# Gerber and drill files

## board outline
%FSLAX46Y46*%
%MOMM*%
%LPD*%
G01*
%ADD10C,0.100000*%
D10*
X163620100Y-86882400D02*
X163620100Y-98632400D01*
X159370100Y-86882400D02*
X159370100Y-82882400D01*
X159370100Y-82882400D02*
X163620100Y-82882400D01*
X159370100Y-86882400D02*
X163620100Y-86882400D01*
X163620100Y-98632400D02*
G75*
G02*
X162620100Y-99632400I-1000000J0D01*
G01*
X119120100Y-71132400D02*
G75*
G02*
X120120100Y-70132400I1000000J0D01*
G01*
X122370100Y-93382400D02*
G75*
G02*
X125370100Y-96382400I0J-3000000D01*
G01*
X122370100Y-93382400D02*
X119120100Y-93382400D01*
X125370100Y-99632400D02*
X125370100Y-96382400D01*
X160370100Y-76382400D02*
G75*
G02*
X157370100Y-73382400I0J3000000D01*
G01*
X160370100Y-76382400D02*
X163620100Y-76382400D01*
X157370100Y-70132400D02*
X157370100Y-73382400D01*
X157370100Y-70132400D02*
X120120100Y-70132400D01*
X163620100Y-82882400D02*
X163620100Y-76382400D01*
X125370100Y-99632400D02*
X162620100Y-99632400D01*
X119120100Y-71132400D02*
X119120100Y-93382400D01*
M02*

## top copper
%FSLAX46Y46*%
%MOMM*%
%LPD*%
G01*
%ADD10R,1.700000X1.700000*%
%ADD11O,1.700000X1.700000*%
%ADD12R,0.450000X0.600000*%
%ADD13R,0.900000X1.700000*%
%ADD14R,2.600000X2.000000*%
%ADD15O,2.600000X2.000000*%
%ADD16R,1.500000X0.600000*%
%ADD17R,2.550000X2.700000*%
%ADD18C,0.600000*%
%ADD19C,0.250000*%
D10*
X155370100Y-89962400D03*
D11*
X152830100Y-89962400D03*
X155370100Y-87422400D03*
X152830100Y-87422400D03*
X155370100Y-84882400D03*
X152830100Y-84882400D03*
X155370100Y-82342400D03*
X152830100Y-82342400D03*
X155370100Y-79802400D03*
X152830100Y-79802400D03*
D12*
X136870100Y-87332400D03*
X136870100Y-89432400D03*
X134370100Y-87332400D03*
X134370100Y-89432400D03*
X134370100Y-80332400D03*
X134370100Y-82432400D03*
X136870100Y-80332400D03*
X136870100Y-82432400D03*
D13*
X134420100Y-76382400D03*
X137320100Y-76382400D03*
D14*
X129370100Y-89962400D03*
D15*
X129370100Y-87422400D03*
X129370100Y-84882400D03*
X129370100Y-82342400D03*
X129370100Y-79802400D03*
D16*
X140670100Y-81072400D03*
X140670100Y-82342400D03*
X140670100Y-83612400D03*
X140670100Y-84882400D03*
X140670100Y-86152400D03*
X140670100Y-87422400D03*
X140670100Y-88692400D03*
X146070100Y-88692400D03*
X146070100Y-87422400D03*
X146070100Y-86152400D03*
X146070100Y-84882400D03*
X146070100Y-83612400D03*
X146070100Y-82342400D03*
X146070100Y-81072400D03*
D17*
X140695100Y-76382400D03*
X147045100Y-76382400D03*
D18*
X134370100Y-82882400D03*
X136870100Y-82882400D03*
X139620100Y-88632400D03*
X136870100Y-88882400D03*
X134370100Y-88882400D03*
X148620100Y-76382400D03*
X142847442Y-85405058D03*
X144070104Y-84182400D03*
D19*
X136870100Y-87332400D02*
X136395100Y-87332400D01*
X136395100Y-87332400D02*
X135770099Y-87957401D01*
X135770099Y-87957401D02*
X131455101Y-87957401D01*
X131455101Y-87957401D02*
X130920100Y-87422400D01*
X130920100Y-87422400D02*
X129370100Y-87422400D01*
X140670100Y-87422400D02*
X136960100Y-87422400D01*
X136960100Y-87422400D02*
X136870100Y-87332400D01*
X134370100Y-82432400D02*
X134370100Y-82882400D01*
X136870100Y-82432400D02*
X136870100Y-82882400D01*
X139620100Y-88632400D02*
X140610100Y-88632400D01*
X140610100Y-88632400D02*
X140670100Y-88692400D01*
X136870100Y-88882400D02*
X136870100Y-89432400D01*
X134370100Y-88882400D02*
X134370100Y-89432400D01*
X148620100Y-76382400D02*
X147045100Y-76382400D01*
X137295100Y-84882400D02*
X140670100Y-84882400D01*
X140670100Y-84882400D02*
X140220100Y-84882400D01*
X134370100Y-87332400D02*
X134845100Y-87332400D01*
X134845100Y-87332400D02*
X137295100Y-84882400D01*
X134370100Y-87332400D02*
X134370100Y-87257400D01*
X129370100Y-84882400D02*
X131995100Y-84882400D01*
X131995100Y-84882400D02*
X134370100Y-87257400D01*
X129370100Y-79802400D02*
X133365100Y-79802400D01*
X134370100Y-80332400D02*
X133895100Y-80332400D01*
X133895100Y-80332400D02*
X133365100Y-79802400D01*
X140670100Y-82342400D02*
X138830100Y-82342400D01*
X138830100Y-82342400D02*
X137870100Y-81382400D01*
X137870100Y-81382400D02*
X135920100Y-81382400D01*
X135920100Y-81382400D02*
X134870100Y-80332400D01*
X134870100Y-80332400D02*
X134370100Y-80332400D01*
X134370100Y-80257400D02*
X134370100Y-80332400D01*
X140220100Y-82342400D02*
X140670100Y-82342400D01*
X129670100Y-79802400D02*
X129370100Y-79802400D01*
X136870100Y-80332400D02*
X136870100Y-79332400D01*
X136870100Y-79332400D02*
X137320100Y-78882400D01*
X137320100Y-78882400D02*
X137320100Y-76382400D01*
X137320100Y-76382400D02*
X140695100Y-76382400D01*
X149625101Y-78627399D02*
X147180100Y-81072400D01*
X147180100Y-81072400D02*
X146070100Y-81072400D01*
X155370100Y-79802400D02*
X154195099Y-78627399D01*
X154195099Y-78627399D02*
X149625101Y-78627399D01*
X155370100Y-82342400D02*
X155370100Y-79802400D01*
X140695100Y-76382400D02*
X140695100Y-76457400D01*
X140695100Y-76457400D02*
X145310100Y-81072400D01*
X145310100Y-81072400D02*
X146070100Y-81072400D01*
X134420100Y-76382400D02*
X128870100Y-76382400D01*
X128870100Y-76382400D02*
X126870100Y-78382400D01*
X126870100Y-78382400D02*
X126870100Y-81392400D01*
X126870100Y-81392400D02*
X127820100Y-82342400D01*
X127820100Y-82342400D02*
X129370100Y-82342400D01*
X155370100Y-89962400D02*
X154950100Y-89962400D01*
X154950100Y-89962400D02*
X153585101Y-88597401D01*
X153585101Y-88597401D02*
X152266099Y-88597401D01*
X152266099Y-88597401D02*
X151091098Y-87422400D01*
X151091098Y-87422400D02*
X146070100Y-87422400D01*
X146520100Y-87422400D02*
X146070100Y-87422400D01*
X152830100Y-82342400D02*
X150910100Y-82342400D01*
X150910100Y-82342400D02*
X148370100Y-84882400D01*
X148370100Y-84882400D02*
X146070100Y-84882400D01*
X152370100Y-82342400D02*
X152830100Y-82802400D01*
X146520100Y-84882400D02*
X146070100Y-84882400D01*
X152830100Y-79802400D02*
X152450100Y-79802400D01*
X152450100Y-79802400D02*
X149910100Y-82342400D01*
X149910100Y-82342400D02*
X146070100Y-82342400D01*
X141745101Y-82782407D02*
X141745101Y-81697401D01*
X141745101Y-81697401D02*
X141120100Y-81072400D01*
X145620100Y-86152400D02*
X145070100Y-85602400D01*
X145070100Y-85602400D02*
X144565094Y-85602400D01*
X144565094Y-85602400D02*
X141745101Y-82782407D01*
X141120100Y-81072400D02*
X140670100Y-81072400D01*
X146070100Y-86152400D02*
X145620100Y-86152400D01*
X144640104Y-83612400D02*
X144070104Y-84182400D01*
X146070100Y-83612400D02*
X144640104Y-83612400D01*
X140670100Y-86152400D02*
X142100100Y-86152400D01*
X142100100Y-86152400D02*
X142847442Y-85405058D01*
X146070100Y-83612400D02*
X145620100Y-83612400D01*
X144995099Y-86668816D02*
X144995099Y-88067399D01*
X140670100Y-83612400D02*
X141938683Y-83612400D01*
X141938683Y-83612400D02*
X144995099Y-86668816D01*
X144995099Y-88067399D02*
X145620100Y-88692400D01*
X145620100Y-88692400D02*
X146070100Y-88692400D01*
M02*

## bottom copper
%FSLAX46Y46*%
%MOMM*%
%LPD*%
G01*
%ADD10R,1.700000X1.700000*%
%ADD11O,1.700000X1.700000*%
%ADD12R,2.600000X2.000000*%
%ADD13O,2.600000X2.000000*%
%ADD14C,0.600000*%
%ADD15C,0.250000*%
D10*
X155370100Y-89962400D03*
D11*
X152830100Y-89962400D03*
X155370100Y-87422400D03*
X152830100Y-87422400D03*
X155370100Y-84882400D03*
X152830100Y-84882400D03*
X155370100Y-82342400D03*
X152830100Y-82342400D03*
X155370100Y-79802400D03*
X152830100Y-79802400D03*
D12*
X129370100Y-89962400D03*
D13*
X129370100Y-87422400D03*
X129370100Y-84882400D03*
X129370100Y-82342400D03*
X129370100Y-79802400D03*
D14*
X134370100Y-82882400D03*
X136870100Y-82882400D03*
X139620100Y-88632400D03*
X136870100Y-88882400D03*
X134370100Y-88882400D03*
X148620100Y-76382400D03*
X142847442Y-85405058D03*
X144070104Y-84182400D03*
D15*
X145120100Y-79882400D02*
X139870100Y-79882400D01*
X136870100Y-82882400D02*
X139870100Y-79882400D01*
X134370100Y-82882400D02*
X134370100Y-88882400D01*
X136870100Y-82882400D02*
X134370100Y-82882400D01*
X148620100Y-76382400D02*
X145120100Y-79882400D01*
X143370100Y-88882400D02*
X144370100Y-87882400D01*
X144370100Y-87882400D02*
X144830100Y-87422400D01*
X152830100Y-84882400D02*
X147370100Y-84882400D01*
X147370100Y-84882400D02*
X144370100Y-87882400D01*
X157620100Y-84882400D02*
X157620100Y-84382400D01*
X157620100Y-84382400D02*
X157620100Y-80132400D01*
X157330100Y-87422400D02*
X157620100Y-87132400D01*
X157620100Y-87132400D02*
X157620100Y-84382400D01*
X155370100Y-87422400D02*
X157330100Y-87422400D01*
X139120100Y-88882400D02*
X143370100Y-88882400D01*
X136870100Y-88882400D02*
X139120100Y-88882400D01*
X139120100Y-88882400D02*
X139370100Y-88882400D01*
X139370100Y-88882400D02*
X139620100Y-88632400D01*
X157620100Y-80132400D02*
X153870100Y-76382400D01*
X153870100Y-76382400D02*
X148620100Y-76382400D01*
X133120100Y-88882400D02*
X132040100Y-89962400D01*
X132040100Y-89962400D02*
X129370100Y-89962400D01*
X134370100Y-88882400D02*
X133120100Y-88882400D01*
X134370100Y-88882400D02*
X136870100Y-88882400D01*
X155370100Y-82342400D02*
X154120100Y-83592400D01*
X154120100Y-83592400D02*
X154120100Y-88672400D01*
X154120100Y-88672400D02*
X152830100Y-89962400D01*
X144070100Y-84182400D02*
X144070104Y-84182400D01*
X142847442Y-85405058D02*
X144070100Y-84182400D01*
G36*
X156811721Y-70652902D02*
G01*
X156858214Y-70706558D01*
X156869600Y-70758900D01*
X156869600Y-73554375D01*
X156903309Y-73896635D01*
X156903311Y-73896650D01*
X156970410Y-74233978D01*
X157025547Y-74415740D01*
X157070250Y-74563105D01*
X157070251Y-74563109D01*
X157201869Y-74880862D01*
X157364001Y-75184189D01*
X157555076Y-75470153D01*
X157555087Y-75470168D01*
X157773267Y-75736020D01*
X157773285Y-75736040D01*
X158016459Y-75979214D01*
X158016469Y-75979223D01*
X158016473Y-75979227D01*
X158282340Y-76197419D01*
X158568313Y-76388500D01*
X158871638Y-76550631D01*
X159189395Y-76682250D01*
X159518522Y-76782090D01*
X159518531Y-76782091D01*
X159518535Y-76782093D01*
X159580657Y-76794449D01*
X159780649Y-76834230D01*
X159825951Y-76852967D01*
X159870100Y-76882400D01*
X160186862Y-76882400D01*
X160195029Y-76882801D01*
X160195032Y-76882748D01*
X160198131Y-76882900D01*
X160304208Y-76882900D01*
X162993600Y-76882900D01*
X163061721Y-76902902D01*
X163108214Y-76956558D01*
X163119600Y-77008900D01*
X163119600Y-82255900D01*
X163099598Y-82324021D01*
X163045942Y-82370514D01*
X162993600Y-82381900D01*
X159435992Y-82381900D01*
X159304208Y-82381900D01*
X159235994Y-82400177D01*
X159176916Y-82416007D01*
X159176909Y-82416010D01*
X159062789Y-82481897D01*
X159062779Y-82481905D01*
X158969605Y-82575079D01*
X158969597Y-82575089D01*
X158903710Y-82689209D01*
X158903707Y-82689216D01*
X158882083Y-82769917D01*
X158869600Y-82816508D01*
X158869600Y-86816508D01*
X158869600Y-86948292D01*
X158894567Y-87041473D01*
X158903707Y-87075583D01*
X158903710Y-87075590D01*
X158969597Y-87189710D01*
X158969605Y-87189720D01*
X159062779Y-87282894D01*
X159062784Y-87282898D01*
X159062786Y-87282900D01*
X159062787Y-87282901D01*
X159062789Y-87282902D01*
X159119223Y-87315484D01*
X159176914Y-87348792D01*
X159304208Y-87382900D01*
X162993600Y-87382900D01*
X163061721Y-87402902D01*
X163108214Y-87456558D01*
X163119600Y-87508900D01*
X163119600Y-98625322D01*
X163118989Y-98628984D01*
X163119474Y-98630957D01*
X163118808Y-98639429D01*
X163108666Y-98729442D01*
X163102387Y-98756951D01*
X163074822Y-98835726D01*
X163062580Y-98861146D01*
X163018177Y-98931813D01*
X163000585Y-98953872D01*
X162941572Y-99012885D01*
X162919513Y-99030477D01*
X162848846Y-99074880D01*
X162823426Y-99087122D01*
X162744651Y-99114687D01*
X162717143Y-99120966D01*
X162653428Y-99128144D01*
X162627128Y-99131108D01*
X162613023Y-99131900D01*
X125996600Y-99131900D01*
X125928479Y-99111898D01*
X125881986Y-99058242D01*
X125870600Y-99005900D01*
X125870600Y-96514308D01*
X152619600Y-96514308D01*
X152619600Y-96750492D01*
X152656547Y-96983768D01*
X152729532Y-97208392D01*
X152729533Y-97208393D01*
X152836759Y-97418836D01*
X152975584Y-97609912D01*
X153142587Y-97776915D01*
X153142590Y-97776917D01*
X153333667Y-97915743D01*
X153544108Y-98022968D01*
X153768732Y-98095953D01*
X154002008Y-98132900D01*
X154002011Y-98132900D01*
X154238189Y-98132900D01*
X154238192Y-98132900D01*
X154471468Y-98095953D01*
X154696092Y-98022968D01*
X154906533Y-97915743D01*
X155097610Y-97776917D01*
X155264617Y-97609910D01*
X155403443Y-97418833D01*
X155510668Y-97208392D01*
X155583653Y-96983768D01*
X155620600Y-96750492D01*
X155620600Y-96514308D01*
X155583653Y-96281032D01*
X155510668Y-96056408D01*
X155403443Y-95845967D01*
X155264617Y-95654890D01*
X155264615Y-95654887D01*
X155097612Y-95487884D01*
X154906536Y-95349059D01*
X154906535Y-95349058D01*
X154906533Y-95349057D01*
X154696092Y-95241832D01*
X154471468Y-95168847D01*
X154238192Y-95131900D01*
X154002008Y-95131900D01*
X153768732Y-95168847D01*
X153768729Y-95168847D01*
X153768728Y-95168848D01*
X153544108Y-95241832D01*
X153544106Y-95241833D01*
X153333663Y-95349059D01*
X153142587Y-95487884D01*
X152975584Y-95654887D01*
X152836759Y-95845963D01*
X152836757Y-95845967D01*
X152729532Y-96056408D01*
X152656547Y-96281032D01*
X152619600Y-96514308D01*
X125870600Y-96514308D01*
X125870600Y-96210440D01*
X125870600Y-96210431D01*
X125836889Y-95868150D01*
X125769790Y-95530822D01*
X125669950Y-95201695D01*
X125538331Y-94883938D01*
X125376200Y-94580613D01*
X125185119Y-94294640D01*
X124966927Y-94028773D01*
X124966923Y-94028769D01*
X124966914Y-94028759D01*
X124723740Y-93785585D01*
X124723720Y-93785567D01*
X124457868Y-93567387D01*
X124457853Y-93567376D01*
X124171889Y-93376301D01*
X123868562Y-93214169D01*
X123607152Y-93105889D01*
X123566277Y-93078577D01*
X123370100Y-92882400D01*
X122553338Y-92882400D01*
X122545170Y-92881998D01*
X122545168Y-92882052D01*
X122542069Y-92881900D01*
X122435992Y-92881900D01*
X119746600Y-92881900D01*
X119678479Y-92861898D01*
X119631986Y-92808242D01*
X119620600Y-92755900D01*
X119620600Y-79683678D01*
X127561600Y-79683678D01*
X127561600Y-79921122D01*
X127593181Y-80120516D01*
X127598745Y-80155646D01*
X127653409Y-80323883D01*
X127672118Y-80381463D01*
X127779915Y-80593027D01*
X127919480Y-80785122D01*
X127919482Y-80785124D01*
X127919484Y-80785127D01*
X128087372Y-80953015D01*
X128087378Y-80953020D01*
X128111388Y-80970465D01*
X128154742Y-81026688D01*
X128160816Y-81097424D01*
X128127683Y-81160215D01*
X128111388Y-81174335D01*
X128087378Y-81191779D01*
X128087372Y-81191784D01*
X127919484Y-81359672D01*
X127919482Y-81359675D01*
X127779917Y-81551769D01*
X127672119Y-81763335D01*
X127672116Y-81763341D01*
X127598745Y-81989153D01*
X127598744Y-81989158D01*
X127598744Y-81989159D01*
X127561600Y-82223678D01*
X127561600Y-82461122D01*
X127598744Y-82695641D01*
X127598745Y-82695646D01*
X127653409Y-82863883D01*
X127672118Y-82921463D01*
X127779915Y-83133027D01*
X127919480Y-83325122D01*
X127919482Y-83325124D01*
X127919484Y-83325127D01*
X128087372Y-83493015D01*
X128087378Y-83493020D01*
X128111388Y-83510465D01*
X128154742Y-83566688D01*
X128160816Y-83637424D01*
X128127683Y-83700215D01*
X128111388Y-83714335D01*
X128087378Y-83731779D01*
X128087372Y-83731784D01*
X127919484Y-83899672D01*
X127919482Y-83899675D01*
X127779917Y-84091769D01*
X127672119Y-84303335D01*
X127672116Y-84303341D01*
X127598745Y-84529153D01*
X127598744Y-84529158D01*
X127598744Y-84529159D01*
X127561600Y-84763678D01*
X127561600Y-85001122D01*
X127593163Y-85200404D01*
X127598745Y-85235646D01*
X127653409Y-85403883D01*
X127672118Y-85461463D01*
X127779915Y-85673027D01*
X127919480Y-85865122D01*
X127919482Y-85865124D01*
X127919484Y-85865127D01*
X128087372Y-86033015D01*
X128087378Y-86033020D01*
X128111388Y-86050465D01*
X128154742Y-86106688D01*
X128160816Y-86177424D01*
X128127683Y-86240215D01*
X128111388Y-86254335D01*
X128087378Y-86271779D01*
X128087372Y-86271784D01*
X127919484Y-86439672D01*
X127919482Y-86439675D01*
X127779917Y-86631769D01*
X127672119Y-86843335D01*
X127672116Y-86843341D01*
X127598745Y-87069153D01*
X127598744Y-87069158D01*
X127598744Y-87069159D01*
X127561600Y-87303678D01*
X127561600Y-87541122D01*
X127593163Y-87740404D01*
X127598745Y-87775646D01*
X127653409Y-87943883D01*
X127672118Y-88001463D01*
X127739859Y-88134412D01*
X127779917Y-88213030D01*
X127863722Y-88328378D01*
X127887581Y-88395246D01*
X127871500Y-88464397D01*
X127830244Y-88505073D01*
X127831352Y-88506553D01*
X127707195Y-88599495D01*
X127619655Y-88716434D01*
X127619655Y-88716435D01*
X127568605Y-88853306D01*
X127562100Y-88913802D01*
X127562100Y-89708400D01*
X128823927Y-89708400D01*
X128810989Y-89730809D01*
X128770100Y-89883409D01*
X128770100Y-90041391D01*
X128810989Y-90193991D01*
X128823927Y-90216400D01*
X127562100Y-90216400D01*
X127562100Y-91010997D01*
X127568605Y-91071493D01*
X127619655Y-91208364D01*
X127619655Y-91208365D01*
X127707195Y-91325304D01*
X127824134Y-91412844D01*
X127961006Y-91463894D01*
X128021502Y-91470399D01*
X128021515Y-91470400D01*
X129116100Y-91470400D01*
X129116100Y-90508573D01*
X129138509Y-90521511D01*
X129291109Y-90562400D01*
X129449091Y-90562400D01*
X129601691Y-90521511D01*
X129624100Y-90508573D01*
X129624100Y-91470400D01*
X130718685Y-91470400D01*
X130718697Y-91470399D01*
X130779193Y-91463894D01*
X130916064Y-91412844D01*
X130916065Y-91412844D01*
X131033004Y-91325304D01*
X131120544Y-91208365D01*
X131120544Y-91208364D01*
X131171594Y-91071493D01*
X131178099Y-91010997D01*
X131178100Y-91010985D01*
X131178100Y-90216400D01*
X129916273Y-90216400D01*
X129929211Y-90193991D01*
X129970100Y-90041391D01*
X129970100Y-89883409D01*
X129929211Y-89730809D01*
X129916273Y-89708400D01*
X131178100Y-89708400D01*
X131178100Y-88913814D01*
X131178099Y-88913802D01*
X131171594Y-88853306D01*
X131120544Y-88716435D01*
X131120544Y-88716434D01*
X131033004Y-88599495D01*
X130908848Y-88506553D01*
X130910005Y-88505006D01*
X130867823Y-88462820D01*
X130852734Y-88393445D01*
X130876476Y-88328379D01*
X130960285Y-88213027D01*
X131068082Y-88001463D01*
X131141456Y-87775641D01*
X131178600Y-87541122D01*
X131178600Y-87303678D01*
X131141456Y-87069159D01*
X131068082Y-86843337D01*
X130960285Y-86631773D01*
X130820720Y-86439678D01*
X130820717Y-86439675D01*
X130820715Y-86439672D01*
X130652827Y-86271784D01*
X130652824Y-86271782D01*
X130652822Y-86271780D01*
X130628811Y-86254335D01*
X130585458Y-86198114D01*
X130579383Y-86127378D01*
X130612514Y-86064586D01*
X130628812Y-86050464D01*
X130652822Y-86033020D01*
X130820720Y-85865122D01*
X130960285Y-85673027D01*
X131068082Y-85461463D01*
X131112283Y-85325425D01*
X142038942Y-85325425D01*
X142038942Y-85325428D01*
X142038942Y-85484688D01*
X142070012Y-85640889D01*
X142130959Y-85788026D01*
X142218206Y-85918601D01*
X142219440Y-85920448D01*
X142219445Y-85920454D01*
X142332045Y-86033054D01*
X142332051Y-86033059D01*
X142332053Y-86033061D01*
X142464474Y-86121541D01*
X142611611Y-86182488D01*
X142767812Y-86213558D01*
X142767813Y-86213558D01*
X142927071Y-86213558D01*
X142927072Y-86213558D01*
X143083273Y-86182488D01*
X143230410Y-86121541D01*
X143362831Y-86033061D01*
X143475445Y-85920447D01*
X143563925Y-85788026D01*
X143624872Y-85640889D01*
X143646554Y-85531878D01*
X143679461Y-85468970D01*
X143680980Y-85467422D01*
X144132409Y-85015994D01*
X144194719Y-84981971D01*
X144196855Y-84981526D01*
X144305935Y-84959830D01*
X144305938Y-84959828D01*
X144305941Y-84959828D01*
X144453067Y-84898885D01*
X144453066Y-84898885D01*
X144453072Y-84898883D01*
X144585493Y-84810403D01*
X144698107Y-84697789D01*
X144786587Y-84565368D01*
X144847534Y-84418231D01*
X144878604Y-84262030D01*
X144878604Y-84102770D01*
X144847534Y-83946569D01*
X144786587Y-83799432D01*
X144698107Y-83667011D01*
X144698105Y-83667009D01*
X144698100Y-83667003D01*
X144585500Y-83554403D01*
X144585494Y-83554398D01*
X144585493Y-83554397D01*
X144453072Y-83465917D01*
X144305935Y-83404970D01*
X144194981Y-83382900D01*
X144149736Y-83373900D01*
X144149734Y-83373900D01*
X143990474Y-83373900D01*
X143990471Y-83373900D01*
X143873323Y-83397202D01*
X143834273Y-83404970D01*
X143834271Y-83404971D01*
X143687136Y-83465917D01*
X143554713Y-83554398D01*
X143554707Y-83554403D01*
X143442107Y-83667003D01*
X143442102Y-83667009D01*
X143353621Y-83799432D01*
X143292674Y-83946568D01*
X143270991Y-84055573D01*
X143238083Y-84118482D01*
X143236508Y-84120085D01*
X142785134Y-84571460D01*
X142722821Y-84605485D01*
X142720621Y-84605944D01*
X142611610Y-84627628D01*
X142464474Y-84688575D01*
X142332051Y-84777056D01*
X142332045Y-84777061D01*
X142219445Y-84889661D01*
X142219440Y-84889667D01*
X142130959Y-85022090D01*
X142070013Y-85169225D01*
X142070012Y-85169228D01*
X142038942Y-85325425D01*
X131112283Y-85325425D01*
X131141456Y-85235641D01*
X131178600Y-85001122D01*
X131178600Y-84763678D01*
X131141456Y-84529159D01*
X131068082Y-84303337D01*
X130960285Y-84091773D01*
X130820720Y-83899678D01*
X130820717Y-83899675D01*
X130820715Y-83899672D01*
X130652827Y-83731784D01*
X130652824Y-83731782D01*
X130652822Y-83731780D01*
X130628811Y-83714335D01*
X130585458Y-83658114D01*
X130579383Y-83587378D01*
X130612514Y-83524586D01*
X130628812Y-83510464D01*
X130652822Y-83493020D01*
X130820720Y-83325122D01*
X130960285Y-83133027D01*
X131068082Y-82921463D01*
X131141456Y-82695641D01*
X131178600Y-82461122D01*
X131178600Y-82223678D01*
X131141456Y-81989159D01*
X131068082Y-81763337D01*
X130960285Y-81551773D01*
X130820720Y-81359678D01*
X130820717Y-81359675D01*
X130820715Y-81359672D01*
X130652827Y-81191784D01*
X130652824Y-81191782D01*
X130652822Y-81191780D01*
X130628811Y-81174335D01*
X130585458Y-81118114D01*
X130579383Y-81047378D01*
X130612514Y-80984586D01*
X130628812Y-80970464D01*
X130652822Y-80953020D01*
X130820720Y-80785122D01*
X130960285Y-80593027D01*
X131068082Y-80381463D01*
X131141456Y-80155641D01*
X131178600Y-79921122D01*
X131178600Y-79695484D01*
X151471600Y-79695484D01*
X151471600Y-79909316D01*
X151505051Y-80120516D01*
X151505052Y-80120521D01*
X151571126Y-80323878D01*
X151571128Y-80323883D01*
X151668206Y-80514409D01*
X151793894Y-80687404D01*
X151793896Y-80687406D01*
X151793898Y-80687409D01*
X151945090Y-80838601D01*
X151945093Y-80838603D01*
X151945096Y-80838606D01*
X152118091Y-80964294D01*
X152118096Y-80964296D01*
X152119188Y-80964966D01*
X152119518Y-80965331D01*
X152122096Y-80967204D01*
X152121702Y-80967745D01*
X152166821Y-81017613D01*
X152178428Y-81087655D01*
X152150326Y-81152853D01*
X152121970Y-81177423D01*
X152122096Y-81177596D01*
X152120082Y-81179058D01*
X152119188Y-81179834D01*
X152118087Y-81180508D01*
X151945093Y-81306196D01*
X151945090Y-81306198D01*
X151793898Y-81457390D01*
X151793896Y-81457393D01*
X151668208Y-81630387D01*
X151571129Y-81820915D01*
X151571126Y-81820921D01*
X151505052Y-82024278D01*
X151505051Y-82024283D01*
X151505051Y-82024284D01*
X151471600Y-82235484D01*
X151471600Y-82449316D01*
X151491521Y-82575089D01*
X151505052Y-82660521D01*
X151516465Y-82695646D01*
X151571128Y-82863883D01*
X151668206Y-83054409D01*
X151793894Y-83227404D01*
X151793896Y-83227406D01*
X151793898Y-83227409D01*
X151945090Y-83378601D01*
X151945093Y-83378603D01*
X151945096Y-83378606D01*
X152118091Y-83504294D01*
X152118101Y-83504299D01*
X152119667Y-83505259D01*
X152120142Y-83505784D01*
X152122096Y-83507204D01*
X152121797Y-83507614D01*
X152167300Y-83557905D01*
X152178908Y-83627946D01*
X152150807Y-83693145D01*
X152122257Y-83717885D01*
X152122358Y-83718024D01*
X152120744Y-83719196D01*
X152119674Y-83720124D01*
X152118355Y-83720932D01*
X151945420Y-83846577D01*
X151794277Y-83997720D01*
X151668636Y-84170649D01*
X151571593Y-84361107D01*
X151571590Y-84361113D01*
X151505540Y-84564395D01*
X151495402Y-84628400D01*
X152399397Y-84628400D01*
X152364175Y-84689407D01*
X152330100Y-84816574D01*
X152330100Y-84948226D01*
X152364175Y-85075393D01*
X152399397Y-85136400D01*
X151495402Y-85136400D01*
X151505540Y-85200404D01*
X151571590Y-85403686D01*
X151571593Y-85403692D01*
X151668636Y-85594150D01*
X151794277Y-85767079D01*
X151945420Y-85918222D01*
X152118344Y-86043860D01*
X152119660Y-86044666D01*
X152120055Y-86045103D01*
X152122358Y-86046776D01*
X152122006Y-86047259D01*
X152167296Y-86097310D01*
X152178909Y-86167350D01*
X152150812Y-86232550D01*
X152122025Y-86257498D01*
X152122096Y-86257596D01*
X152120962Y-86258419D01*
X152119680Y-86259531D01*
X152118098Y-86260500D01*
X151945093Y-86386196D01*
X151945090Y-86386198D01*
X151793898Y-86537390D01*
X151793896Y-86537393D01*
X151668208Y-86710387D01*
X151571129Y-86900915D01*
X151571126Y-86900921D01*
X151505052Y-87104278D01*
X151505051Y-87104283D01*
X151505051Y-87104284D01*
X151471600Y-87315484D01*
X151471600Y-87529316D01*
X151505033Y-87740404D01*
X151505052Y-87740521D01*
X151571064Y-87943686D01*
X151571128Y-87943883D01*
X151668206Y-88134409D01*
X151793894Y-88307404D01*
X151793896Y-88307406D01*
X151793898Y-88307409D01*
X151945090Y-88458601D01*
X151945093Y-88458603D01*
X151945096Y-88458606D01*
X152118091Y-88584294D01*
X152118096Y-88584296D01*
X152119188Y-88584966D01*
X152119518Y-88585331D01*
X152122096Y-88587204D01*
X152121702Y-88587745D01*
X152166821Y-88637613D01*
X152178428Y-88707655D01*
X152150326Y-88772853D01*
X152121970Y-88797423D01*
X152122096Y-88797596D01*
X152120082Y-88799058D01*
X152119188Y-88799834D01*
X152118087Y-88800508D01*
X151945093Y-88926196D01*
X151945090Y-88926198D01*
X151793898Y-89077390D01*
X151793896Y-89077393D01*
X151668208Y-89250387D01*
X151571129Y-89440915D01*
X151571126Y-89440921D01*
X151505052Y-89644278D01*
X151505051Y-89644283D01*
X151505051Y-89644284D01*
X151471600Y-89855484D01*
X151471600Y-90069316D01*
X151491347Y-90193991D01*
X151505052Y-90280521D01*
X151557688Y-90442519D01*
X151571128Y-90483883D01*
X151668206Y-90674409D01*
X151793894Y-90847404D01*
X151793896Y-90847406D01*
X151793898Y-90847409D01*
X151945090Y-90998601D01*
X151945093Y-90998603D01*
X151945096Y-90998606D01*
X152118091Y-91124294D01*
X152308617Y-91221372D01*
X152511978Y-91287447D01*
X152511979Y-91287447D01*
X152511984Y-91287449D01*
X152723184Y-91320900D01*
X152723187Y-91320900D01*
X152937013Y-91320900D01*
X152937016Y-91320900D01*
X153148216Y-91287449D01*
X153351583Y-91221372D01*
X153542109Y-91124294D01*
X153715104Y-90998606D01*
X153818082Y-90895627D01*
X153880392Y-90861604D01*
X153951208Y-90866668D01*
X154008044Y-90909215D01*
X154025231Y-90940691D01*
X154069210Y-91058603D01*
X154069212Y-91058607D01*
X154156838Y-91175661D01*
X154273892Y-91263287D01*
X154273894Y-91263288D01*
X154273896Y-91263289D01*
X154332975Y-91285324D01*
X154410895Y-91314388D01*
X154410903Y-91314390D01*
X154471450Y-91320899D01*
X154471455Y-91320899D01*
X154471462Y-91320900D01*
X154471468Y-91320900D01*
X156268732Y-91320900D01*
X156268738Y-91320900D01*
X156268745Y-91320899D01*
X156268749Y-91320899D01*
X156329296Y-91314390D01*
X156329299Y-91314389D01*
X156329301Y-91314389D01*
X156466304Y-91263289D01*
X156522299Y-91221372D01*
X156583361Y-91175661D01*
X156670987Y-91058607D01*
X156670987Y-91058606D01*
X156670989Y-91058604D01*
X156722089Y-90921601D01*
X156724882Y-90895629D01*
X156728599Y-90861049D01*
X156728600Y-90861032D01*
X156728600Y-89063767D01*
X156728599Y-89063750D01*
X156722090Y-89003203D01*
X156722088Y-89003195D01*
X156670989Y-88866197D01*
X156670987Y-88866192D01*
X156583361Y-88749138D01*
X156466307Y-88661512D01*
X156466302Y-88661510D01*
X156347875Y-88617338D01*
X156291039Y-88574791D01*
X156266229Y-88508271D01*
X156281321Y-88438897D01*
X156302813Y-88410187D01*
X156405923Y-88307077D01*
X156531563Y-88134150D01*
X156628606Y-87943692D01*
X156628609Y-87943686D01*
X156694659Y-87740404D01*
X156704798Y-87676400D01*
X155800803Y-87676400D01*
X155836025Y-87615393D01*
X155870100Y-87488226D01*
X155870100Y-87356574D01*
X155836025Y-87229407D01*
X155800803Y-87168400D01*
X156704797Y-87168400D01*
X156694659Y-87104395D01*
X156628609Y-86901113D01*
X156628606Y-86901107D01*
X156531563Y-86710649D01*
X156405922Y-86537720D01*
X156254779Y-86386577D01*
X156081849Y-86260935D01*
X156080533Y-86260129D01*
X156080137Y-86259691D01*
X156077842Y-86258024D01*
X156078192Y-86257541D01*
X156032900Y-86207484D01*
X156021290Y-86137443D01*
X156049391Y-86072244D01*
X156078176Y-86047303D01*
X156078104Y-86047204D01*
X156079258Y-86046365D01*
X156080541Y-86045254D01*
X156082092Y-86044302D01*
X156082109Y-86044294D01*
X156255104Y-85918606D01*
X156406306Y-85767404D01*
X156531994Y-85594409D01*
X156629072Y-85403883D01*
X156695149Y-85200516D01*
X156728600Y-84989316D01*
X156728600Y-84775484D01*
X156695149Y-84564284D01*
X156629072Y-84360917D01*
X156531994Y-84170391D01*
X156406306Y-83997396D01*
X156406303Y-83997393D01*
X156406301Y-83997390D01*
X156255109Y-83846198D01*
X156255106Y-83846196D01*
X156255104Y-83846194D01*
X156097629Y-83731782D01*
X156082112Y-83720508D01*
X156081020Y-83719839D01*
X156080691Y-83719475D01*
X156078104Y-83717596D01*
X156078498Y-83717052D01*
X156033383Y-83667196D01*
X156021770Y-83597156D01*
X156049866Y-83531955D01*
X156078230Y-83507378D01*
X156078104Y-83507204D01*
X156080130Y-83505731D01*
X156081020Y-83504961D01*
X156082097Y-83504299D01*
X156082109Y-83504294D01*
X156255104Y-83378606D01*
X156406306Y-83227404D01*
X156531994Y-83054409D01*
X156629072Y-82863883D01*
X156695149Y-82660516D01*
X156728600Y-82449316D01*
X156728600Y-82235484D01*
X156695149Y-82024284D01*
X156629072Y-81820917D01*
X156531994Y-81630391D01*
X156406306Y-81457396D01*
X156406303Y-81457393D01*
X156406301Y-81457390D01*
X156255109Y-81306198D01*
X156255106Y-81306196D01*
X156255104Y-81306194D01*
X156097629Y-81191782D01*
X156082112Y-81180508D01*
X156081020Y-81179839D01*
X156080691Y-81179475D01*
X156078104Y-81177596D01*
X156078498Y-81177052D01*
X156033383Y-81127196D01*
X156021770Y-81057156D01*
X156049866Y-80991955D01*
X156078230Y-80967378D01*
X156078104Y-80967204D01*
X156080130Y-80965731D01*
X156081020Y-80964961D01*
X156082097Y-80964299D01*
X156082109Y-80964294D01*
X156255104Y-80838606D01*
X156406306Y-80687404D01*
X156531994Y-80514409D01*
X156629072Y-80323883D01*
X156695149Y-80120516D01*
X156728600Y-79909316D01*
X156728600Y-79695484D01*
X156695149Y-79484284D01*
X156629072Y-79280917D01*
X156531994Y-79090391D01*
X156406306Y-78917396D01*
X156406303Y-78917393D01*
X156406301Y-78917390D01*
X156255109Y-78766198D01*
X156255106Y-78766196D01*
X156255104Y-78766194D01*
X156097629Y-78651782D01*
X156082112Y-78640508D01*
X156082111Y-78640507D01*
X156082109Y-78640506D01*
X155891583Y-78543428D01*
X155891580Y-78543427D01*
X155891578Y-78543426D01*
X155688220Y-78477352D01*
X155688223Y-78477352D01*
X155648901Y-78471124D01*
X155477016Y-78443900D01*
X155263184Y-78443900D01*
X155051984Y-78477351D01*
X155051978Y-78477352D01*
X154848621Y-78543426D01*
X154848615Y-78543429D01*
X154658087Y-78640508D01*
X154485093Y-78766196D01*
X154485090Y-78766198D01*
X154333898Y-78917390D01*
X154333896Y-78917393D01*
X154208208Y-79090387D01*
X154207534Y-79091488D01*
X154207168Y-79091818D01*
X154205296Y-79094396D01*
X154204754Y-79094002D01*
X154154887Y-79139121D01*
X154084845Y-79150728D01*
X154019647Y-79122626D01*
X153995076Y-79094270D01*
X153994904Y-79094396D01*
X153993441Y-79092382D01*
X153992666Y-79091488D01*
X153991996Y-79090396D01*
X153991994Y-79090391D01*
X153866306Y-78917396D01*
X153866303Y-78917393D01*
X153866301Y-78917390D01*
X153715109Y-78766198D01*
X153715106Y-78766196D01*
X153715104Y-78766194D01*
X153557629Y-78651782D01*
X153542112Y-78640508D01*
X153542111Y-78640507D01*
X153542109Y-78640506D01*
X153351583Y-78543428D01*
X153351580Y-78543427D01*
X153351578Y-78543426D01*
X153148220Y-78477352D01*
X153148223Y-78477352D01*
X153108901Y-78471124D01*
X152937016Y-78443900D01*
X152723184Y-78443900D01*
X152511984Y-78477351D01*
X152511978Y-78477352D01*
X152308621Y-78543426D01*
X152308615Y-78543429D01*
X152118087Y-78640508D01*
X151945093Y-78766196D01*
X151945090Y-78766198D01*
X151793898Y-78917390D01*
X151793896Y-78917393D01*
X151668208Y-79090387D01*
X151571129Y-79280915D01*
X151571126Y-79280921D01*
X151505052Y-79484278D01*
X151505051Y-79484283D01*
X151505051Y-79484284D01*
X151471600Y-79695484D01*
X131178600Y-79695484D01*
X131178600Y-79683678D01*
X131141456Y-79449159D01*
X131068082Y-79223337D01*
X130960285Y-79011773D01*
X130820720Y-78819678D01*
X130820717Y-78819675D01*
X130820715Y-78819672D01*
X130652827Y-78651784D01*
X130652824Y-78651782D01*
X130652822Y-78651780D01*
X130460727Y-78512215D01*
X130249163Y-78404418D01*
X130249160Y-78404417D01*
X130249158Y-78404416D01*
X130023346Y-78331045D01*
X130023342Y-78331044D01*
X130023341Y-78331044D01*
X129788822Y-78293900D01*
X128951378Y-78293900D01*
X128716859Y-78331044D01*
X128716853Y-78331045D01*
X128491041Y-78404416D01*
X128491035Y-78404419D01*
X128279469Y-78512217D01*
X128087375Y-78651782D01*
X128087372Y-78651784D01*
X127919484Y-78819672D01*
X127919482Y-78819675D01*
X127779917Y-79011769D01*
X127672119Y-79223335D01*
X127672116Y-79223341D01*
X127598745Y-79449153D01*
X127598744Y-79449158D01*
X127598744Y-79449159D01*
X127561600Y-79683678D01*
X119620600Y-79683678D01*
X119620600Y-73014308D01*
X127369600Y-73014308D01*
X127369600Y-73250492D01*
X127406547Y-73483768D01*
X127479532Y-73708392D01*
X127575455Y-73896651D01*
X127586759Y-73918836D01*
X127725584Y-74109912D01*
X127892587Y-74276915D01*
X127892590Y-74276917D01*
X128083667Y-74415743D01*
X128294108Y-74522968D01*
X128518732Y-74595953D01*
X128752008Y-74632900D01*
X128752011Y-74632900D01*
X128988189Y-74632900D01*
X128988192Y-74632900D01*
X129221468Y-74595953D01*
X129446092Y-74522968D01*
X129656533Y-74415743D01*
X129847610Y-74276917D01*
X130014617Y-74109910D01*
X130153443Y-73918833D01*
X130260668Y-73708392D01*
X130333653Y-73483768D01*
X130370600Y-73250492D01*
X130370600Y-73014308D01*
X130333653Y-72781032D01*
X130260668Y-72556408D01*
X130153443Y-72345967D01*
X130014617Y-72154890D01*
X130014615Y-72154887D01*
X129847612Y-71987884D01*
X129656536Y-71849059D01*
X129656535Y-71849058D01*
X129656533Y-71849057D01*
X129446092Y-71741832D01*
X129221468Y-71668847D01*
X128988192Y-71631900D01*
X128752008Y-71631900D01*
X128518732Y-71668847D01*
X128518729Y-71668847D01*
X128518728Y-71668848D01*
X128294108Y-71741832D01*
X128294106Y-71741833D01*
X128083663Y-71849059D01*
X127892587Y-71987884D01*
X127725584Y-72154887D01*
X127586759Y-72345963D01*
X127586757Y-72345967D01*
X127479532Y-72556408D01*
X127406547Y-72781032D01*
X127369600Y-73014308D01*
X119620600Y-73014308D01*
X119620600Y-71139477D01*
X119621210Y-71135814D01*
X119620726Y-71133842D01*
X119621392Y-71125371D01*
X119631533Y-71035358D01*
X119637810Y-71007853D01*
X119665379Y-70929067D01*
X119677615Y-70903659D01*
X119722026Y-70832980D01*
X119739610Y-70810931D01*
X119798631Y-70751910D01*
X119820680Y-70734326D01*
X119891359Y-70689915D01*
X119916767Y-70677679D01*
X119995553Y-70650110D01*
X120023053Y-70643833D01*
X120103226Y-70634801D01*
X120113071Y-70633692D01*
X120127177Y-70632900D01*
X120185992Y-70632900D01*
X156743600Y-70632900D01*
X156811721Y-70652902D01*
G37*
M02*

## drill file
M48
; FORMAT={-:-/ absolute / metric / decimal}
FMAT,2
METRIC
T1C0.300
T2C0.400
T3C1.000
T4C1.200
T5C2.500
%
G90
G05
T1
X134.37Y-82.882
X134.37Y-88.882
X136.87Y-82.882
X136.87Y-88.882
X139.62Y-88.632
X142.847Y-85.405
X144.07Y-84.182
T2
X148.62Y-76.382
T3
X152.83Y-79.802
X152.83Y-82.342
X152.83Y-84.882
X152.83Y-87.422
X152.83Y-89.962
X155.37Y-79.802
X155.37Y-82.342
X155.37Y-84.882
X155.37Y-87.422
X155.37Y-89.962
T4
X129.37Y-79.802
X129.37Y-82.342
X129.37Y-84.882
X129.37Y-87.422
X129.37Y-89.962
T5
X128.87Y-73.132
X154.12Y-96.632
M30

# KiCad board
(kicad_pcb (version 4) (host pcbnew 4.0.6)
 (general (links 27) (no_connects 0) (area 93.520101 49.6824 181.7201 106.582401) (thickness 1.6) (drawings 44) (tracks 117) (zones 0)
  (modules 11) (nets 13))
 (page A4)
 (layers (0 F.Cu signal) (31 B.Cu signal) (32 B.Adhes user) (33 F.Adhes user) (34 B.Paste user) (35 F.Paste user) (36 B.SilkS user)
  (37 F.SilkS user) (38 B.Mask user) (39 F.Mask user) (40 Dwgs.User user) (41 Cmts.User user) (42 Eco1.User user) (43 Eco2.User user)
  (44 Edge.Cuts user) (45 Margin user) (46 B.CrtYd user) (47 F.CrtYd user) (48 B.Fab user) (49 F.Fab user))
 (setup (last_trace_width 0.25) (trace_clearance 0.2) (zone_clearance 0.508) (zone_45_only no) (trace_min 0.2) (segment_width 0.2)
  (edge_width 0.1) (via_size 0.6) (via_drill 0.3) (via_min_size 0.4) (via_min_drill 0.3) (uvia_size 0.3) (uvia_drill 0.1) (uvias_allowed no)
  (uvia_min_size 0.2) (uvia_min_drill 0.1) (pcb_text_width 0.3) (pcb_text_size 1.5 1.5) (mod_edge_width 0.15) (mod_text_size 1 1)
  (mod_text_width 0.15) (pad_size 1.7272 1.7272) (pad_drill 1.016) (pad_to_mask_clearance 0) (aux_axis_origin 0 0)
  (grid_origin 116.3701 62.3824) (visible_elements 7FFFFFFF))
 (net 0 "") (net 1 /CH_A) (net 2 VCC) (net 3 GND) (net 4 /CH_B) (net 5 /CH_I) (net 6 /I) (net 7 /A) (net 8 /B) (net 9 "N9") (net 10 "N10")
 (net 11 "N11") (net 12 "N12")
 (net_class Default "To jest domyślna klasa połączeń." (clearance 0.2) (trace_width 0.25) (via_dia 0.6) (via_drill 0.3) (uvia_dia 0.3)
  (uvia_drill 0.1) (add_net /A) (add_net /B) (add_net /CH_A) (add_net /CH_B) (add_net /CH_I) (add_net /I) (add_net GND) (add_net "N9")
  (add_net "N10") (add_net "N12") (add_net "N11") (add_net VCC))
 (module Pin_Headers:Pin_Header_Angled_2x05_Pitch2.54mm (layer F.Cu) (at 152.8301 79.8024)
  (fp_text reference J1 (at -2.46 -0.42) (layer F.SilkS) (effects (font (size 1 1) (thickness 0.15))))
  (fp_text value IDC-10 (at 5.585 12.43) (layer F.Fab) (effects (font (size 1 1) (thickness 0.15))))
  (pad 1 thru_hole rect (at 2.54 10.16) (size 1.7 1.7) (drill 1) (layers *.Cu *.Mask) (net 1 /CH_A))
  (pad 2 thru_hole oval (at 0 10.16) (size 1.7 1.7) (drill 1) (layers *.Cu *.Mask) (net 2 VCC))
  (pad 3 thru_hole oval (at 2.54 7.62) (size 1.7 1.7) (drill 1) (layers *.Cu *.Mask) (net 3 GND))
  (pad 4 thru_hole oval (at 0 7.62) (size 1.7 1.7) (drill 1) (layers *.Cu *.Mask))
  (pad 5 thru_hole oval (at 2.54 5.08) (size 1.7 1.7) (drill 1) (layers *.Cu *.Mask))
  (pad 6 thru_hole oval (at 0 5.08) (size 1.7 1.7) (drill 1) (layers *.Cu *.Mask) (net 3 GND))
  (pad 7 thru_hole oval (at 2.54 2.54) (size 1.7 1.7) (drill 1) (layers *.Cu *.Mask) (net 2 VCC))
  (pad 8 thru_hole oval (at 0 2.54) (size 1.7 1.7) (drill 1) (layers *.Cu *.Mask) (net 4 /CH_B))
  (pad 9 thru_hole oval (at 2.54 0) (size 1.7 1.7) (drill 1) (layers *.Cu *.Mask) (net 2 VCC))
  (pad 10 thru_hole oval (at 0 0) (size 1.7 1.7) (drill 1) (layers *.Cu *.Mask) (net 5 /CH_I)))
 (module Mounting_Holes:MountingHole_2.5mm (layer F.Cu) (at 128.8701 73.1324)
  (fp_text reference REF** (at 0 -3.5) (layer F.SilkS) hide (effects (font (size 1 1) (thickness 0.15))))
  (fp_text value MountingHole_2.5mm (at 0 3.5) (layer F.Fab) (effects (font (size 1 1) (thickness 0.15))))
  (pad 1 np_thru_hole circle (at 0 0) (size 2.5 2.5) (drill 2.5) (layers *.Cu *.Mask)))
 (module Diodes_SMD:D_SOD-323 (layer F.Cu) (at 136.8701 88.3824 270)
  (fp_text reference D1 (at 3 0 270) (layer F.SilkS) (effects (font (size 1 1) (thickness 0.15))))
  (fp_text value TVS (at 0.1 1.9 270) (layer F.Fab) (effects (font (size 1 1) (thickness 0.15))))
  (pad 1 smd rect (at -1.05 0 270) (size 0.6 0.45) (layers F.Cu F.Paste F.Mask) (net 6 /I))
  (pad 2 smd rect (at 1.05 0 270) (size 0.6 0.45) (layers F.Cu F.Paste F.Mask) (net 3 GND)))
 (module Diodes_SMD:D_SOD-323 (layer F.Cu) (at 134.3701 88.3824 270)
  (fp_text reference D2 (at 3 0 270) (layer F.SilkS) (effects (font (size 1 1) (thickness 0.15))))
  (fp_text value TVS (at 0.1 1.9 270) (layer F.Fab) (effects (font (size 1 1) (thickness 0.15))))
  (pad 1 smd rect (at -1.05 0 270) (size 0.6 0.45) (layers F.Cu F.Paste F.Mask) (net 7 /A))
  (pad 2 smd rect (at 1.05 0 270) (size 0.6 0.45) (layers F.Cu F.Paste F.Mask) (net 3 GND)))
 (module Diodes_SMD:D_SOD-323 (layer F.Cu) (at 134.3701 81.3824 270)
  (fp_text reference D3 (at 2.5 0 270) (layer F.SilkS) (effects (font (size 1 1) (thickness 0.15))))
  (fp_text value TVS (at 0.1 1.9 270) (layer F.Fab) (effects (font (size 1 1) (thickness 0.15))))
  (pad 1 smd rect (at -1.05 0 270) (size 0.6 0.45) (layers F.Cu F.Paste F.Mask) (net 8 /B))
  (pad 2 smd rect (at 1.05 0 270) (size 0.6 0.45) (layers F.Cu F.Paste F.Mask) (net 3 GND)))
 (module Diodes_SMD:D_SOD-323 (layer F.Cu) (at 136.8701 81.3824 270)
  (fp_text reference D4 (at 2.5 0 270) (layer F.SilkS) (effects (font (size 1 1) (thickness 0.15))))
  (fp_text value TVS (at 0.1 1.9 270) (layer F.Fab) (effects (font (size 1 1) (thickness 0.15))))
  (pad 1 smd rect (at -1.05 0 270) (size 0.6 0.45) (layers F.Cu F.Paste F.Mask) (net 2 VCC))
  (pad 2 smd rect (at 1.05 0 270) (size 0.6 0.45) (layers F.Cu F.Paste F.Mask) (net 3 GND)))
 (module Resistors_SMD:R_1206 (layer F.Cu) (at 135.8701 76.3824)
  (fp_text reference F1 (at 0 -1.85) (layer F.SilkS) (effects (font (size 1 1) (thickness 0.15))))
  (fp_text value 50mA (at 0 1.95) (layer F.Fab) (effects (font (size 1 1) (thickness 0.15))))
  (pad 1 smd rect (at -1.45 0) (size 0.9 1.7) (layers F.Cu F.Paste F.Mask) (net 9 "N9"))
  (pad 2 smd rect (at 1.45 0) (size 0.9 1.7) (layers F.Cu F.Paste F.Mask) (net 2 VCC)))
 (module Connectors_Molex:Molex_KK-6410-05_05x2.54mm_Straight (layer F.Cu) (at 129.3701 89.9624 90)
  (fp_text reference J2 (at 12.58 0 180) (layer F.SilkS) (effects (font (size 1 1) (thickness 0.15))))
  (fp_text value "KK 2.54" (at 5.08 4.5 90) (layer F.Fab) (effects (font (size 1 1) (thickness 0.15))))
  (pad 1 thru_hole rect (at 0 0 90) (size 2 2.6) (drill 1.2) (layers *.Cu *.Mask) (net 3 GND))
  (pad 2 thru_hole oval (at 2.54 0 90) (size 2 2.6) (drill 1.2) (layers *.Cu *.Mask) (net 6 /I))
  (pad 3 thru_hole oval (at 5.08 0 90) (size 2 2.6) (drill 1.2) (layers *.Cu *.Mask) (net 7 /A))
  (pad 4 thru_hole oval (at 7.62 0 90) (size 2 2.6) (drill 1.2) (layers *.Cu *.Mask) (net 9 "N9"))
  (pad 5 thru_hole oval (at 10.16 0 90) (size 2 2.6) (drill 1.2) (layers *.Cu *.Mask) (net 8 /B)))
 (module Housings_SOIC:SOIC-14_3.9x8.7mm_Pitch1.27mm (layer F.Cu) (at 143.3701 84.8824)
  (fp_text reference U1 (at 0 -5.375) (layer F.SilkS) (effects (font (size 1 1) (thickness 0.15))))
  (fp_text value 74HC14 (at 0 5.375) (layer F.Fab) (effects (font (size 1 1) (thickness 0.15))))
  (pad 1 smd rect (at -2.7 -3.81) (size 1.5 0.6) (layers F.Cu F.Paste F.Mask) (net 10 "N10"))
  (pad 2 smd rect (at -2.7 -2.54) (size 1.5 0.6) (layers F.Cu F.Paste F.Mask) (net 8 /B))
  (pad 3 smd rect (at -2.7 -1.27) (size 1.5 0.6) (layers F.Cu F.Paste F.Mask) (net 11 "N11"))
  (pad 4 smd rect (at -2.7 0) (size 1.5 0.6) (layers F.Cu F.Paste F.Mask) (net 7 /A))
  (pad 5 smd rect (at -2.7 1.27) (size 1.5 0.6) (layers F.Cu F.Paste F.Mask) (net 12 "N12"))
  (pad 6 smd rect (at -2.7 2.54) (size 1.5 0.6) (layers F.Cu F.Paste F.Mask) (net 6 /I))
  (pad 7 smd rect (at -2.7 3.81) (size 1.5 0.6) (layers F.Cu F.Paste F.Mask) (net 3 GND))
  (pad 8 smd rect (at 2.7 3.81) (size 1.5 0.6) (layers F.Cu F.Paste F.Mask) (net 11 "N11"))
  (pad 9 smd rect (at 2.7 2.54) (size 1.5 0.6) (layers F.Cu F.Paste F.Mask) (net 1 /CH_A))
  (pad 10 smd rect (at 2.7 1.27) (size 1.5 0.6) (layers F.Cu F.Paste F.Mask) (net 10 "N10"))
  (pad 11 smd rect (at 2.7 0) (size 1.5 0.6) (layers F.Cu F.Paste F.Mask) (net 4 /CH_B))
  (pad 12 smd rect (at 2.7 -1.27) (size 1.5 0.6) (layers F.Cu F.Paste F.Mask) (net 12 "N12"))
  (pad 13 smd rect (at 2.7 -2.54) (size 1.5 0.6) (layers F.Cu F.Paste F.Mask) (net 5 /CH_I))
  (pad 14 smd rect (at 2.7 -3.81) (size 1.5 0.6) (layers F.Cu F.Paste F.Mask) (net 2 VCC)))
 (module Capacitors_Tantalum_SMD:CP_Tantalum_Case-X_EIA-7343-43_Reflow (layer F.Cu) (at 143.8701 76.3824)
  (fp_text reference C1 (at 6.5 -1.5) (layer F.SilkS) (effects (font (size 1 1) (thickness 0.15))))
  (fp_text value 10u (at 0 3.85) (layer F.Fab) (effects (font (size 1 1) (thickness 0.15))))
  (pad 1 smd rect (at -3.175 0) (size 2.55 2.7) (layers F.Cu F.Paste F.Mask) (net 2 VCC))
  (pad 2 smd rect (at 3.175 0) (size 2.55 2.7) (layers F.Cu F.Paste F.Mask) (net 3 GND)))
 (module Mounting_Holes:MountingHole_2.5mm (layer F.Cu) (at 154.1201 96.6324)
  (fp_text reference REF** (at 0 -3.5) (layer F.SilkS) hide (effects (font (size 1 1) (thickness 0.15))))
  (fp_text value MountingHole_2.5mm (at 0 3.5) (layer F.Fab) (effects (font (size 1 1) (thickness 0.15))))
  (pad 1 np_thru_hole circle (at 0 0) (size 2.5 2.5) (drill 2.5) (layers *.Cu *.Mask)))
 (gr_line (start 163.6201 86.8824) (end 163.6201 98.6324) (layer Edge.Cuts) (width 0.1))
 (gr_line (start 159.3701 86.8824) (end 159.3701 82.8824) (layer Edge.Cuts) (width 0.1))
 (gr_line (start 159.3701 82.8824) (end 163.6201 82.8824) (layer Edge.Cuts) (width 0.1))
 (gr_line (start 159.3701 86.8824) (end 163.6201 86.8824) (layer Edge.Cuts) (width 0.1))
 (gr_arc (start 162.6201 98.6324) (end 163.6201 98.6324) (angle 90) (layer Edge.Cuts) (width 0.1))
 (gr_arc (start 120.1201 71.1324) (end 119.1201 71.1324) (angle 90) (layer Edge.Cuts) (width 0.1))
 (gr_arc (start 122.3701 96.3824) (end 122.3701 93.3824) (angle 90) (layer Edge.Cuts) (width 0.1))
 (gr_line (start 122.3701 93.3824) (end 119.1201 93.3824) (layer Edge.Cuts) (width 0.1))
 (gr_line (start 125.3701 99.6324) (end 125.3701 96.3824) (layer Edge.Cuts) (width 0.1))
 (gr_arc (start 160.3701 73.3824) (end 160.3701 76.3824) (angle 90) (layer Edge.Cuts) (width 0.1))
 (gr_line (start 160.3701 76.3824) (end 163.6201 76.3824) (layer Edge.Cuts) (width 0.1))
 (gr_line (start 157.3701 70.1324) (end 157.3701 73.3824) (layer Edge.Cuts) (width 0.1))
 (gr_line (start 157.3701 70.1324) (end 120.1201 70.1324) (layer Edge.Cuts) (width 0.1))
 (gr_line (start 163.6201 82.8824) (end 163.6201 76.3824) (layer Edge.Cuts) (width 0.1))
 (gr_line (start 125.3701 99.6324) (end 162.6201 99.6324) (layer Edge.Cuts) (width 0.1))
 (gr_line (start 119.1201 71.1324) (end 119.1201 93.3824) (layer Edge.Cuts) (width 0.1))
 (segment (start 136.8701 87.3324) (end 136.3951 87.3324) (width 0.25) (layer F.Cu) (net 6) (status 10))
 (segment (start 136.3951 87.3324) (end 135.770099 87.957401) (width 0.25) (layer F.Cu) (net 6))
 (segment (start 135.770099 87.957401) (end 131.455101 87.957401) (width 0.25) (layer F.Cu) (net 6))
 (segment (start 131.455101 87.957401) (end 130.9201 87.4224) (width 0.25) (layer F.Cu) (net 6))
 (segment (start 130.9201 87.4224) (end 129.3701 87.4224) (width 0.25) (layer F.Cu) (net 6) (status 20))
 (segment (start 140.6701 87.4224) (end 136.9601 87.4224) (width 0.25) (layer F.Cu) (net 6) (status 30))
 (segment (start 136.9601 87.4224) (end 136.8701 87.3324) (width 0.25) (layer F.Cu) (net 6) (status 30))
 (segment (start 145.1201 79.8824) (end 139.8701 79.8824) (width 0.25) (layer B.Cu) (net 3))
 (segment (start 136.8701 82.8824) (end 139.8701 79.8824) (width 0.25) (layer B.Cu) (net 3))
 (segment (start 134.3701 82.4324) (end 134.3701 82.8824) (width 0.25) (layer F.Cu) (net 3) (status 10))
 (via (at 134.3701 82.8824) (size 0.6) (drill 0.3) (layers F.Cu B.Cu) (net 3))
 (segment (start 134.3701 82.8824) (end 134.3701 88.8824) (width 0.25) (layer B.Cu) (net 3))
 (segment (start 136.8701 82.8824) (end 134.3701 82.8824) (width 0.25) (layer B.Cu) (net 3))
 (segment (start 136.8701 82.4324) (end 136.8701 82.8824) (width 0.25) (layer F.Cu) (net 3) (status 10))
 (via (at 136.8701 82.8824) (size 0.6) (drill 0.3) (layers F.Cu B.Cu) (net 3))
 (segment (start 148.6201 76.3824) (end 145.1201 79.8824) (width 0.25) (layer B.Cu) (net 3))
 (segment (start 143.3701 88.8824) (end 144.3701 87.8824) (width 0.25) (layer B.Cu) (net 3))
 (segment (start 144.3701 87.8824) (end 144.8301 87.4224) (width 0.25) (layer B.Cu) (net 3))
 (segment (start 152.8301 84.8824) (end 147.3701 84.8824) (width 0.25) (layer B.Cu) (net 3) (status 10))
 (segment (start 147.3701 84.8824) (end 144.3701 87.8824) (width 0.25) (layer B.Cu) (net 3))
 (segment (start 157.6201 84.8824) (end 157.6201 84.3824) (width 0.25) (layer B.Cu) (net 3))
 (segment (start 157.6201 84.3824) (end 157.6201 80.1324) (width 0.25) (layer B.Cu) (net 3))
 (segment (start 157.3301 87.4224) (end 157.6201 87.1324) (width 0.25) (layer B.Cu) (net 3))
 (segment (start 157.6201 87.1324) (end 157.6201 84.3824) (width 0.25) (layer B.Cu) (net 3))
 (segment (start 155.3701 87.4224) (end 157.3301 87.4224) (width 0.25) (layer B.Cu) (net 3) (status 10))
 (segment (start 139.6201 88.6324) (end 140.6101 88.6324) (width 0.25) (layer F.Cu) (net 3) (status 20))
 (segment (start 140.6101 88.6324) (end 140.6701 88.6924) (width 0.25) (layer F.Cu) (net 3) (status 30))
 (segment (start 139.1201 88.8824) (end 143.3701 88.8824) (width 0.25) (layer B.Cu) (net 3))
 (segment (start 136.8701 88.8824) (end 139.1201 88.8824) (width 0.25) (layer B.Cu) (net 3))
 (segment (start 139.1201 88.8824) (end 139.3701 88.8824) (width 0.25) (layer B.Cu) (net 3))
 (segment (start 139.3701 88.8824) (end 139.6201 88.6324) (width 0.25) (layer B.Cu) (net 3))
 (via (at 139.6201 88.6324) (size 0.6) (drill 0.3) (layers F.Cu B.Cu) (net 3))
 (segment (start 157.6201 80.1324) (end 153.8701 76.3824) (width 0.25) (layer B.Cu) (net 3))
 (segment (start 153.8701 76.3824) (end 148.6201 76.3824) (width 0.25) (layer B.Cu) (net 3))
 (segment (start 133.1201 88.8824) (end 132.0401 89.9624) (width 0.25) (layer B.Cu) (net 3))
 (segment (start 132.0401 89.9624) (end 129.3701 89.9624) (width 0.25) (layer B.Cu) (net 3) (status 20))
 (segment (start 134.3701 88.8824) (end 133.1201 88.8824) (width 0.25) (layer B.Cu) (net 3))
 (segment (start 136.8701 88.8824) (end 136.8701 89.4324) (width 0.25) (layer F.Cu) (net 3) (status 20))
 (segment (start 134.3701 88.8824) (end 136.8701 88.8824) (width 0.25) (layer B.Cu) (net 3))
 (via (at 136.8701 88.8824) (size 0.6) (drill 0.3) (layers F.Cu B.Cu) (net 3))
 (segment (start 134.3701 88.8824) (end 134.3701 89.4324) (width 0.25) (layer F.Cu) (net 3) (status 20))
 (via (at 134.3701 88.8824) (size 0.6) (drill 0.3) (layers F.Cu B.Cu) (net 3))
 (segment (start 148.6201 76.3824) (end 147.0451 76.3824) (width 0.25) (layer F.Cu) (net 3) (status 20))
 (via (at 148.6201 76.3824) (size 0.6) (drill 0.4) (layers F.Cu B.Cu) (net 3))
 (segment (start 137.2951 84.8824) (end 140.6701 84.8824) (width 0.25) (layer F.Cu) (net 7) (status 20))
 (segment (start 140.6701 84.8824) (end 140.2201 84.8824) (width 0.25) (layer F.Cu) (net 7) (status 30))
 (segment (start 134.3701 87.3324) (end 134.8451 87.3324) (width 0.25) (layer F.Cu) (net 7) (status 10))
 (segment (start 134.8451 87.3324) (end 137.2951 84.8824) (width 0.25) (layer F.Cu) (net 7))
 (segment (start 134.3701 87.3324) (end 134.3701 87.2574) (width 0.25) (layer F.Cu) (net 7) (status 30))
 (segment (start 129.3701 84.8824) (end 131.9951 84.8824) (width 0.25) (layer F.Cu) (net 7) (status 10))
 (segment (start 131.9951 84.8824) (end 134.3701 87.2574) (width 0.25) (layer F.Cu) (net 7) (status 20))
 (segment (start 129.3701 79.8024) (end 133.3651 79.8024) (width 0.25) (layer F.Cu) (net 8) (status 10))
 (segment (start 134.3701 80.3324) (end 133.8951 80.3324) (width 0.25) (layer F.Cu) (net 8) (status 10))
 (segment (start 133.8951 80.3324) (end 133.3651 79.8024) (width 0.25) (layer F.Cu) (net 8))
 (segment (start 140.6701 82.3424) (end 138.8301 82.3424) (width 0.25) (layer F.Cu) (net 8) (status 10))
 (segment (start 138.8301 82.3424) (end 137.8701 81.3824) (width 0.25) (layer F.Cu) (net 8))
 (segment (start 137.8701 81.3824) (end 135.9201 81.3824) (width 0.25) (layer F.Cu) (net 8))
 (segment (start 135.9201 81.3824) (end 134.8701 80.3324) (width 0.25) (layer F.Cu) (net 8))
 (segment (start 134.8701 80.3324) (end 134.3701 80.3324) (width 0.25) (layer F.Cu) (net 8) (status 20))
 (segment (start 134.3701 80.2574) (end 134.3701 80.3324) (width 0.25) (layer F.Cu) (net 8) (status 30))
 (segment (start 140.2201 82.3424) (end 140.6701 82.3424) (width 0.25) (layer F.Cu) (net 8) (status 30))
 (segment (start 129.6701 79.8024) (end 129.3701 79.8024) (width 0.25) (layer F.Cu) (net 8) (status 30))
 (segment (start 155.3701 82.3424) (end 154.1201 83.5924) (width 0.25) (layer B.Cu) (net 2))
 (segment (start 154.1201 83.5924) (end 154.1201 88.6724) (width 0.25) (layer B.Cu) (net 2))
 (segment (start 154.1201 88.6724) (end 152.8301 89.9624) (width 0.25) (layer B.Cu) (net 2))
 (segment (start 136.8701 80.3324) (end 136.8701 79.3324) (width 0.25) (layer F.Cu) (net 2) (status 10))
 (segment (start 136.8701 79.3324) (end 137.3201 78.8824) (width 0.25) (layer F.Cu) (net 2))
 (segment (start 137.3201 78.8824) (end 137.3201 76.3824) (width 0.25) (layer F.Cu) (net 2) (status 20))
 (segment (start 137.3201 76.3824) (end 140.6951 76.3824) (width 0.25) (layer F.Cu) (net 2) (status 30))
 (segment (start 149.625101 78.627399) (end 147.1801 81.0724) (width 0.25) (layer F.Cu) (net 2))
 (segment (start 147.1801 81.0724) (end 146.0701 81.0724) (width 0.25) (layer F.Cu) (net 2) (status 20))
 (segment (start 155.3701 79.8024) (end 154.195099 78.627399) (width 0.25) (layer F.Cu) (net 2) (status 10))
 (segment (start 154.195099 78.627399) (end 149.625101 78.627399) (width 0.25) (layer F.Cu) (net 2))
 (segment (start 155.3701 82.3424) (end 155.3701 79.8024) (width 0.25) (layer F.Cu) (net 2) (status 30))
 (segment (start 140.6951 76.3824) (end 140.6951 76.4574) (width 0.25) (layer F.Cu) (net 2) (status 30))
 (segment (start 140.6951 76.4574) (end 145.3101 81.0724) (width 0.25) (layer F.Cu) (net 2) (status 10))
 (segment (start 145.3101 81.0724) (end 146.0701 81.0724) (width 0.25) (layer F.Cu) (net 2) (status 20))
 (segment (start 134.4201 76.3824) (end 128.8701 76.3824) (width 0.25) (layer F.Cu) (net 9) (status 10))
 (segment (start 128.8701 76.3824) (end 126.8701 78.3824) (width 0.25) (layer F.Cu) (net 9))
 (segment (start 126.8701 78.3824) (end 126.8701 81.3924) (width 0.25) (layer F.Cu) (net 9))
 (segment (start 126.8701 81.3924) (end 127.8201 82.3424) (width 0.25) (layer F.Cu) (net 9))
 (segment (start 127.8201 82.3424) (end 129.3701 82.3424) (width 0.25) (layer F.Cu) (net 9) (status 20))
 (segment (start 155.3701 89.9624) (end 154.9501 89.9624) (width 0.25) (layer F.Cu) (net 1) (status 30))
 (segment (start 154.9501 89.9624) (end 153.585101 88.597401) (width 0.25) (layer F.Cu) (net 1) (status 10))
 (segment (start 153.585101 88.597401) (end 152.266099 88.597401) (width 0.25) (layer F.Cu) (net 1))
 (segment (start 152.266099 88.597401) (end 151.091098 87.4224) (width 0.25) (layer F.Cu) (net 1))
 (segment (start 151.091098 87.4224) (end 146.0701 87.4224) (width 0.25) (layer F.Cu) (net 1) (status 20))
 (segment (start 146.5201 87.4224) (end 146.0701 87.4224) (width 0.25) (layer F.Cu) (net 1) (status 30))
 (segment (start 152.8301 82.3424) (end 150.9101 82.3424) (width 0.25) (layer F.Cu) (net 4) (status 10))
 (segment (start 150.9101 82.3424) (end 148.3701 84.8824) (width 0.25) (layer F.Cu) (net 4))
 (segment (start 148.3701 84.8824) (end 146.0701 84.8824) (width 0.25) (layer F.Cu) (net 4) (status 20))
 (segment (start 152.3701 82.3424) (end 152.8301 82.8024) (width 0.25) (layer F.Cu) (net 4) (status 30))
 (segment (start 146.5201 84.8824) (end 146.0701 84.8824) (width 0.25) (layer F.Cu) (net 4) (status 30))
 (segment (start 152.8301 79.8024) (end 152.4501 79.8024) (width 0.25) (layer F.Cu) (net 5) (status 30))
 (segment (start 152.4501 79.8024) (end 149.9101 82.3424) (width 0.25) (layer F.Cu) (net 5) (status 10))
 (segment (start 149.9101 82.3424) (end 146.0701 82.3424) (width 0.25) (layer F.Cu) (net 5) (status 20))
 (segment (start 141.745101 82.782407) (end 141.745101 81.697401) (width 0.25) (layer F.Cu) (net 10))
 (segment (start 141.745101 81.697401) (end 141.1201 81.0724) (width 0.25) (layer F.Cu) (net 10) (status 20))
 (segment (start 145.6201 86.1524) (end 145.0701 85.6024) (width 0.25) (layer F.Cu) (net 10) (status 10))
 (segment (start 145.0701 85.6024) (end 144.565094 85.6024) (width 0.25) (layer F.Cu) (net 10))
 (segment (start 144.565094 85.6024) (end 141.745101 82.782407) (width 0.25) (layer F.Cu) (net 10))
 (segment (start 141.1201 81.0724) (end 140.6701 81.0724) (width 0.25) (layer F.Cu) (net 10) (status 30))
 (segment (start 146.0701 86.1524) (end 145.6201 86.1524) (width 0.25) (layer F.Cu) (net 10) (status 30))
 (segment (start 144.0701 84.1824) (end 144.070104 84.1824) (width 0.25) (layer B.Cu) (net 12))
 (segment (start 142.847442 85.405058) (end 144.0701 84.1824) (width 0.25) (layer B.Cu) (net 12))
 (segment (start 144.640104 83.6124) (end 144.070104 84.1824) (width 0.25) (layer F.Cu) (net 12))
 (segment (start 146.0701 83.6124) (end 144.640104 83.6124) (width 0.25) (layer F.Cu) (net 12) (status 10))
 (via (at 142.847442 85.405058) (size 0.6) (drill 0.3) (layers F.Cu B.Cu) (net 12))
 (segment (start 140.6701 86.1524) (end 142.1001 86.1524) (width 0.25) (layer F.Cu) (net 12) (status 10))
 (segment (start 142.1001 86.1524) (end 142.847442 85.405058) (width 0.25) (layer F.Cu) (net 12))
 (via (at 144.070104 84.1824) (size 0.6) (drill 0.3) (layers F.Cu B.Cu) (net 12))
 (segment (start 146.0701 83.6124) (end 145.6201 83.6124) (width 0.25) (layer F.Cu) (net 12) (status 30))
 (segment (start 144.995099 86.668816) (end 144.995099 88.067399) (width 0.25) (layer F.Cu) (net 11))
 (segment (start 140.6701 83.6124) (end 141.938683 83.6124) (width 0.25) (layer F.Cu) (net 11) (status 10))
 (segment (start 141.938683 83.6124) (end 144.995099 86.668816) (width 0.25) (layer F.Cu) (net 11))
 (segment (start 144.995099 88.067399) (end 145.6201 88.6924) (width 0.25) (layer F.Cu) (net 11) (status 20))
 (segment (start 145.6201 88.6924) (end 146.0701 88.6924) (width 0.25) (layer F.Cu) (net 11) (status 30))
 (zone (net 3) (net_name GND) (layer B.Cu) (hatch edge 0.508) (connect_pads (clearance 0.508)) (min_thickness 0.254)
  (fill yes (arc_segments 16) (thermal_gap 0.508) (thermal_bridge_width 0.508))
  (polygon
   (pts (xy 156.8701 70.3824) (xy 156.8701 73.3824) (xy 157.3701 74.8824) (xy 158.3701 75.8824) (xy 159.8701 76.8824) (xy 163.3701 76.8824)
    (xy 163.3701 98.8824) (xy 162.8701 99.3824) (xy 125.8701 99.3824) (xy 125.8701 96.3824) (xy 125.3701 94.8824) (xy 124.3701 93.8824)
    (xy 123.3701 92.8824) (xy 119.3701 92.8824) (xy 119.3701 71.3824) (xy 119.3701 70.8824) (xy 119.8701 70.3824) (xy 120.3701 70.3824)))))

